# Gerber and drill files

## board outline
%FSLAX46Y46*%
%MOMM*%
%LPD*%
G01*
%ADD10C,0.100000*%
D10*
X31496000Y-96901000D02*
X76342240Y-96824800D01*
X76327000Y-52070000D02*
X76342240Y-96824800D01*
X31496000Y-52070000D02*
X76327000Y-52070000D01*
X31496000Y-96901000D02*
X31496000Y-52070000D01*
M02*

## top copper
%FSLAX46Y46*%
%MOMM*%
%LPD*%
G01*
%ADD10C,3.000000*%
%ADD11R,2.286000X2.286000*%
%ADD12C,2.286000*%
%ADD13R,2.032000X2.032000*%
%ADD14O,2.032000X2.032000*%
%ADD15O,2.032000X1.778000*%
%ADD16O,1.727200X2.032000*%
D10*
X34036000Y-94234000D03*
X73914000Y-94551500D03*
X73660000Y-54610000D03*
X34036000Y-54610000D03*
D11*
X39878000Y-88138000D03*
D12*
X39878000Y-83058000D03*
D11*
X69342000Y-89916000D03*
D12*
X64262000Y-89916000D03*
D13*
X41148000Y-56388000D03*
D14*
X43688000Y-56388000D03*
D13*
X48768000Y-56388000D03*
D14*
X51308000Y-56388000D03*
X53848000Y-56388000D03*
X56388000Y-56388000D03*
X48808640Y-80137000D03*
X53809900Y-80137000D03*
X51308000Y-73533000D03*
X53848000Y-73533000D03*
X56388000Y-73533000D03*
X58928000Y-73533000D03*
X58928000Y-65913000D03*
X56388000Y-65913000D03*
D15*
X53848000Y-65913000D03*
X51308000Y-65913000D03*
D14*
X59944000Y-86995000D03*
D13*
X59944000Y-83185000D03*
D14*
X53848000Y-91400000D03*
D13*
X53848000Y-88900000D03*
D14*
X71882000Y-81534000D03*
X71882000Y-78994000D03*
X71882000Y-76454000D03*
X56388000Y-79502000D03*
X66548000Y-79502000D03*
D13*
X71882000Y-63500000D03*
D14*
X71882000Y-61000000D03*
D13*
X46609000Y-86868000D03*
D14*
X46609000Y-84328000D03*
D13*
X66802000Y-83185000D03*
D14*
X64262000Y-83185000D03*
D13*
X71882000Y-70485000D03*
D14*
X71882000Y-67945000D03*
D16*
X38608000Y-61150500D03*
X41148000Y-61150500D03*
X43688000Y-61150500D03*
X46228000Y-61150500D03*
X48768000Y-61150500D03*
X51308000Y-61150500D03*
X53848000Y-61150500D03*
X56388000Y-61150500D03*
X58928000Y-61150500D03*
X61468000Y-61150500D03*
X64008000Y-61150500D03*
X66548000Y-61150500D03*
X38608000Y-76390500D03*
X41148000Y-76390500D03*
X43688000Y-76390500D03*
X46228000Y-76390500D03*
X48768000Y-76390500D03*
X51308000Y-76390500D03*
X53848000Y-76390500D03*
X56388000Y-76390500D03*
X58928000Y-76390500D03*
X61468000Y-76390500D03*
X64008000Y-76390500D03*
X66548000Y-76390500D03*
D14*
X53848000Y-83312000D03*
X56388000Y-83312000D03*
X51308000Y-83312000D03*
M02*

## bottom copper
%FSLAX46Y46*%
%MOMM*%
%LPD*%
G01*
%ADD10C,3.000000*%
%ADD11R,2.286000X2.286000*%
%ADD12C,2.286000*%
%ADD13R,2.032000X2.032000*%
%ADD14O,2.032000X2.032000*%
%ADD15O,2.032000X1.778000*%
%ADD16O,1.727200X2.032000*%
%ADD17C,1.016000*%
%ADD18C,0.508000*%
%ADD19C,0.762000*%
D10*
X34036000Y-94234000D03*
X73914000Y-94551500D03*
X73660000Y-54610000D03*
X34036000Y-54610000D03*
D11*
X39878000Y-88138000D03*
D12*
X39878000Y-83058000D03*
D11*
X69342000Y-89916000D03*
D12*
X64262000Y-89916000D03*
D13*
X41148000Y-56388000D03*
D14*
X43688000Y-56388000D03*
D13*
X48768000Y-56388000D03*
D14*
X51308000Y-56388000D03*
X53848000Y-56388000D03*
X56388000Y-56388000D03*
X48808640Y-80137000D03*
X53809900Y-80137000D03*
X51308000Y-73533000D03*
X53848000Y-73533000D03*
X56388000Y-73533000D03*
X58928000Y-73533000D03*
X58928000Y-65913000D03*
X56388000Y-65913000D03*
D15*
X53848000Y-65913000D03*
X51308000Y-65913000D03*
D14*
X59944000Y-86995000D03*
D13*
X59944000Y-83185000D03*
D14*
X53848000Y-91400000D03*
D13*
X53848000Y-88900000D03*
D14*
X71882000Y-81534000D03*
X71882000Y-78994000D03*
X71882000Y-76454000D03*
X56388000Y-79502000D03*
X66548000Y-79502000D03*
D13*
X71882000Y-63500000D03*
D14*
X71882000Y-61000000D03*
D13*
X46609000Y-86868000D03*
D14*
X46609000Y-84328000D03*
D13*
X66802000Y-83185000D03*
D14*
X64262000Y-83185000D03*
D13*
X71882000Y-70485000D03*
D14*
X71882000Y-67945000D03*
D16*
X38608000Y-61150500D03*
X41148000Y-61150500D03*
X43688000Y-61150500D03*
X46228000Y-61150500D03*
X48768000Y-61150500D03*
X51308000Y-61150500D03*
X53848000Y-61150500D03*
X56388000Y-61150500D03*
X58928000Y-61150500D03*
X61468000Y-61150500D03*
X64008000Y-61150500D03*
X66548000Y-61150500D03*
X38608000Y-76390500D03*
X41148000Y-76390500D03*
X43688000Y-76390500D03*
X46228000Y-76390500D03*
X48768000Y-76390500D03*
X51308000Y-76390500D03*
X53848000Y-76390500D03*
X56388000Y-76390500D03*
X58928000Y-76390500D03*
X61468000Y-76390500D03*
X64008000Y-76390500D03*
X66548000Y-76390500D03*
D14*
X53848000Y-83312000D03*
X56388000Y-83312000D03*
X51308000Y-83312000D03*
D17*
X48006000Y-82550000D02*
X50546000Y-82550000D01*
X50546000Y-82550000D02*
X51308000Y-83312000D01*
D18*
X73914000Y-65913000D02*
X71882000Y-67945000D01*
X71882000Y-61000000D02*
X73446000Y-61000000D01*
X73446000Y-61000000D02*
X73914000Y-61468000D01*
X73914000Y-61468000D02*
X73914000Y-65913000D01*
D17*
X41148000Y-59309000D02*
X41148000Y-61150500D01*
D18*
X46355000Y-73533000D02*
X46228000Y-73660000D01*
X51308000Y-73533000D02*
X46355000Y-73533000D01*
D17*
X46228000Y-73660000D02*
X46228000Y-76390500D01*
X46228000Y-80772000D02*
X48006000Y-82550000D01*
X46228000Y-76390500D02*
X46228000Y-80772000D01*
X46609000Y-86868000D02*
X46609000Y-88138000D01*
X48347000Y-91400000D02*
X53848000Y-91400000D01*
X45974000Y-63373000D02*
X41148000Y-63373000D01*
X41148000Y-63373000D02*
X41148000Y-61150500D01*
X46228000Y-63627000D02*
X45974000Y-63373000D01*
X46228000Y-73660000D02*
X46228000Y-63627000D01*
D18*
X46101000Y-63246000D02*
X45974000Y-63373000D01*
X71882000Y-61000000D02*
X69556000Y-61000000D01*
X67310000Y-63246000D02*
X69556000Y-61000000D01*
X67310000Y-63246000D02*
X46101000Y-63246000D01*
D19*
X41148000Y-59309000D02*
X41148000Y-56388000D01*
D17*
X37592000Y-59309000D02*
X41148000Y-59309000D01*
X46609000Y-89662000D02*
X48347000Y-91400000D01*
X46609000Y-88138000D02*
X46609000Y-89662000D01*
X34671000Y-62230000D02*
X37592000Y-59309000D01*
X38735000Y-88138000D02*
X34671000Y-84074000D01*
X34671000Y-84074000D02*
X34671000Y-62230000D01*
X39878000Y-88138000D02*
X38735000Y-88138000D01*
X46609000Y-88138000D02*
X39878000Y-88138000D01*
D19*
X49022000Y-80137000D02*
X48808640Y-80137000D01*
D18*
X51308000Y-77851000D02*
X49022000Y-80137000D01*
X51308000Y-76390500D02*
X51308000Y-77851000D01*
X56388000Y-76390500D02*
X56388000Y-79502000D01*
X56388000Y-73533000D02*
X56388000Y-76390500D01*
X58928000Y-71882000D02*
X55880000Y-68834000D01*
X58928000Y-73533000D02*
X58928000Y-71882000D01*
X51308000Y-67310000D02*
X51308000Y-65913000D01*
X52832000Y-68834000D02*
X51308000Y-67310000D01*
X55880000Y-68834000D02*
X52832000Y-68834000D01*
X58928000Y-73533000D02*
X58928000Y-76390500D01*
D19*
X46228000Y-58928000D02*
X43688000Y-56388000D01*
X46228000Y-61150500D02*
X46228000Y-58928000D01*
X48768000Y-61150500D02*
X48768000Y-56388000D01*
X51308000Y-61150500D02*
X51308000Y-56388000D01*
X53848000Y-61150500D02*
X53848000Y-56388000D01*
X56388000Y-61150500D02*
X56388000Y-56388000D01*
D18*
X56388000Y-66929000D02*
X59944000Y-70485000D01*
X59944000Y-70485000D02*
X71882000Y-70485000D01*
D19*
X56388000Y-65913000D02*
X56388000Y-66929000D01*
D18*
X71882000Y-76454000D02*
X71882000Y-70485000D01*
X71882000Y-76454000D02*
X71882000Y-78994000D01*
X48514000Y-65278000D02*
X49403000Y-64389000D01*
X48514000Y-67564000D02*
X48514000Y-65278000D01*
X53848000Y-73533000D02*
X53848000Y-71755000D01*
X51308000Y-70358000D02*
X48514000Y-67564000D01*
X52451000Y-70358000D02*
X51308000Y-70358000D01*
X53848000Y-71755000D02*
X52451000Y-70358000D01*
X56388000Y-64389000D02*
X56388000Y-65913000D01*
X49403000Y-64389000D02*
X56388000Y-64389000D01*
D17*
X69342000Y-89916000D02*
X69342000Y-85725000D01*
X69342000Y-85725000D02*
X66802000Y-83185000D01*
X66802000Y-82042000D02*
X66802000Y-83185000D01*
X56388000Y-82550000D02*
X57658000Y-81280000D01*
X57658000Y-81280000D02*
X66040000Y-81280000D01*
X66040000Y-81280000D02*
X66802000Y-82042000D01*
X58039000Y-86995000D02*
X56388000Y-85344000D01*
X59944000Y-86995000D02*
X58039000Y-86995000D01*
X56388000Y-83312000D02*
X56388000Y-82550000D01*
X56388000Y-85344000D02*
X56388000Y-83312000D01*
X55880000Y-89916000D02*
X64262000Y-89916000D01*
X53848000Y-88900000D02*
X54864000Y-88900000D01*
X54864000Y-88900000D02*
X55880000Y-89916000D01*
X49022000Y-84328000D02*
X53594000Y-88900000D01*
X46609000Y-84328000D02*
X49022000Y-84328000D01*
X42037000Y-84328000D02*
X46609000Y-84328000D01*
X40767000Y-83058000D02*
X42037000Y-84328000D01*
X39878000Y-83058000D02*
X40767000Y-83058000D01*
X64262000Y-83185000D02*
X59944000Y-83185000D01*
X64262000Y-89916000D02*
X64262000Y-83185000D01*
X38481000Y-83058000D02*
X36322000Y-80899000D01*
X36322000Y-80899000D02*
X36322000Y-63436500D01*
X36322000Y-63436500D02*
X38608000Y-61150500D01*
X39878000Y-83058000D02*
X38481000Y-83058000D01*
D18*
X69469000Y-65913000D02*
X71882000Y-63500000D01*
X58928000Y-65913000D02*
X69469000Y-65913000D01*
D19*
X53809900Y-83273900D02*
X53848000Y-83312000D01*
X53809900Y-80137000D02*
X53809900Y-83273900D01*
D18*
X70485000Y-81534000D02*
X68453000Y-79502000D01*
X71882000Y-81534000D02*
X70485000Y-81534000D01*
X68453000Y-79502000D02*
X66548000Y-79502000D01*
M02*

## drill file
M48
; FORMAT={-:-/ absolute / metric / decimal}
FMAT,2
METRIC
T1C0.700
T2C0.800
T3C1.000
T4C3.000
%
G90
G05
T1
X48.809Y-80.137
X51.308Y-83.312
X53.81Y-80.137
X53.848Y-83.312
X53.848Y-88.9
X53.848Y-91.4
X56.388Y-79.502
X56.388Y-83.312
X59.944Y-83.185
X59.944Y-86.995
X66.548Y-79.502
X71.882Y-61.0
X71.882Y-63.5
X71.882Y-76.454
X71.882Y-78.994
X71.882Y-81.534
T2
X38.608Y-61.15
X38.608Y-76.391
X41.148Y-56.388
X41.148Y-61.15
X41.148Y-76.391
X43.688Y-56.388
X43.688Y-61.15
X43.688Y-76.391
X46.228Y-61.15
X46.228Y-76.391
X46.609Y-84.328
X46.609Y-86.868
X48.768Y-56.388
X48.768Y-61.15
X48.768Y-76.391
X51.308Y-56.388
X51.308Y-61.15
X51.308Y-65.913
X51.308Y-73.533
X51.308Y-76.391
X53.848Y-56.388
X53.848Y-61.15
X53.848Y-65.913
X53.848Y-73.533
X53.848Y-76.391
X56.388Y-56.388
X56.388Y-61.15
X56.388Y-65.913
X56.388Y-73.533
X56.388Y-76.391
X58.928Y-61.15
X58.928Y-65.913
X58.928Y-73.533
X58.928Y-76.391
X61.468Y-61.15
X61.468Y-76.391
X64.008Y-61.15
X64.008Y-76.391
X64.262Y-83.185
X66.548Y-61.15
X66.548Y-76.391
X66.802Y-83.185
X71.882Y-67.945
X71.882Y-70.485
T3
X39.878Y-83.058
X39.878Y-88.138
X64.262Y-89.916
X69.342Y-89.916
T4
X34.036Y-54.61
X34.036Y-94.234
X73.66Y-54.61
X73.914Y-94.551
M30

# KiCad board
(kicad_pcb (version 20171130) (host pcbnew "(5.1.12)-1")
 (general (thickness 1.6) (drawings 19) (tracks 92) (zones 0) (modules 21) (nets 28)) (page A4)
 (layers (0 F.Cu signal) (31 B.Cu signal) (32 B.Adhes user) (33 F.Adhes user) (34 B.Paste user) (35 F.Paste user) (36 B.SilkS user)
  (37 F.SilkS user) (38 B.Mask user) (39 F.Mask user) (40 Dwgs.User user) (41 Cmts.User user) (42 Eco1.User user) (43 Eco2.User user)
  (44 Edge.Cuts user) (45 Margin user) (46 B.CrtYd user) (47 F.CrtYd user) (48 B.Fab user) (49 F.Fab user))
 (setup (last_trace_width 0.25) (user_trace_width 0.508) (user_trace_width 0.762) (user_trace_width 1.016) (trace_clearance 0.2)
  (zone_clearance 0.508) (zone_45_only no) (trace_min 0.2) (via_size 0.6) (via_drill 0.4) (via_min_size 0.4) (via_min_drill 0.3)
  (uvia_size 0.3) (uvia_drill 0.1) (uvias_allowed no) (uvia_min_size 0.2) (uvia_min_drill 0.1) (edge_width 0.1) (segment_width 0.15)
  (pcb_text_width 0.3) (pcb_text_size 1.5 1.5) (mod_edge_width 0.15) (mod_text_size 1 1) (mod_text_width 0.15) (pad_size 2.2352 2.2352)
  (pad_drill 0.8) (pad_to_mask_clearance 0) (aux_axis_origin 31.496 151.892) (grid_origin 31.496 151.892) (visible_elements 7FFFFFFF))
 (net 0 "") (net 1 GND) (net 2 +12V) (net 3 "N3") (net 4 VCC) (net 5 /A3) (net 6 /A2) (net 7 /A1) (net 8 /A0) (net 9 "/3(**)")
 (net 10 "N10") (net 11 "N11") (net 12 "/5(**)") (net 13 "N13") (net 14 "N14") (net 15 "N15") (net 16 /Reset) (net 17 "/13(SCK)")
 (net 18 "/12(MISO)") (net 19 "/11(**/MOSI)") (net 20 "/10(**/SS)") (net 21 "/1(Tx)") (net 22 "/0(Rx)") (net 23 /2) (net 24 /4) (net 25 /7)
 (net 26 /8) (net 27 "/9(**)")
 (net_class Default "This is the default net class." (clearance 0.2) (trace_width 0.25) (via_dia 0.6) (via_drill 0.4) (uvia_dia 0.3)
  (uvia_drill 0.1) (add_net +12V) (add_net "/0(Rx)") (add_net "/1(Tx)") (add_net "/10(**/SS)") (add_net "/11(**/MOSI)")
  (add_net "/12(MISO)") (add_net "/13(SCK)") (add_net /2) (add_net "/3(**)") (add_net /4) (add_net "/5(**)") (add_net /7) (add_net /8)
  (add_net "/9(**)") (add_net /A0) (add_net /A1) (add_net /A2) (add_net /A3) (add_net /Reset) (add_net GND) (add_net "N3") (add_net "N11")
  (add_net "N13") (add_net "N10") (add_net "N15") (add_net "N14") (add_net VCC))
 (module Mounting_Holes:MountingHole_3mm (layer F.Cu) (at 34.036 94.234)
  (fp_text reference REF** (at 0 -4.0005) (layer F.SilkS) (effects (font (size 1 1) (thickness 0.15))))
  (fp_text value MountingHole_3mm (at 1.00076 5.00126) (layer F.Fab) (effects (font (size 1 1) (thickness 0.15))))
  (pad 1 thru_hole circle (at 0 0) (size 3 3) (drill 3) (layers)))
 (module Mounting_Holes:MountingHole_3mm (layer F.Cu) (at 73.914 94.5515)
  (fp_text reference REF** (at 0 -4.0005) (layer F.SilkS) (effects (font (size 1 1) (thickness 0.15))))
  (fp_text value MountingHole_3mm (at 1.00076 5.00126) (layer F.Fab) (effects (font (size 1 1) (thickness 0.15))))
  (pad 1 thru_hole circle (at 0 0) (size 3 3) (drill 3) (layers)))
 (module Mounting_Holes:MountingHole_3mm (layer F.Cu) (at 73.66 54.61)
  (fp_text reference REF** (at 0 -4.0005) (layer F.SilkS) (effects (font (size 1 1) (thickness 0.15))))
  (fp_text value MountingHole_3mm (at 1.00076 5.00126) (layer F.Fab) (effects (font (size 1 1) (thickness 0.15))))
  (pad 1 thru_hole circle (at 0 0) (size 3 3) (drill 3) (layers)))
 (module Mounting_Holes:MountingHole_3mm (layer F.Cu) (at 34.036 54.61)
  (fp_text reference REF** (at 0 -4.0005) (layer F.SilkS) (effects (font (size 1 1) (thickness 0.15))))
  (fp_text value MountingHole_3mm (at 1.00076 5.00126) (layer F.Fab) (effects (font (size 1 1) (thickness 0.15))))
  (pad 1 thru_hole circle (at 0 0) (size 3 3) (drill 3) (layers)))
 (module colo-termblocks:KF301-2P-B (layer F.Cu) (at 39.878 85.598 90)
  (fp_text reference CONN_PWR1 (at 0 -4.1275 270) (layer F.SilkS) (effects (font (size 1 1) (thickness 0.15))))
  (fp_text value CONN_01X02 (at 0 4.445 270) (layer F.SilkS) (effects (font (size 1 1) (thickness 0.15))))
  (pad 1 thru_hole rect (at -2.54 0 90) (size 2.286 2.286) (drill 1) (layers B.Cu B.Mask) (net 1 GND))
  (pad 2 thru_hole circle (at 2.54 0 90) (size 2.286 2.286) (drill 1) (layers B.Cu B.Mask) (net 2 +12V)))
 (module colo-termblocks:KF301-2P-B (layer F.Cu) (at 66.802 89.916 180)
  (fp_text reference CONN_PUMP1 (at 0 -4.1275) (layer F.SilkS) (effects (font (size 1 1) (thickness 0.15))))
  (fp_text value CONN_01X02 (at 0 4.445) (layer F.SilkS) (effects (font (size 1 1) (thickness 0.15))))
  (pad 1 thru_hole rect (at -2.54 0 180) (size 2.286 2.286) (drill 1) (layers B.Cu B.Mask) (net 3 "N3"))
  (pad 2 thru_hole circle (at 2.54 0 180) (size 2.286 2.286) (drill 1) (layers B.Cu B.Mask) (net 2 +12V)))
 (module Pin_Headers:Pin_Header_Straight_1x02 (layer F.Cu) (at 41.148 56.388 90)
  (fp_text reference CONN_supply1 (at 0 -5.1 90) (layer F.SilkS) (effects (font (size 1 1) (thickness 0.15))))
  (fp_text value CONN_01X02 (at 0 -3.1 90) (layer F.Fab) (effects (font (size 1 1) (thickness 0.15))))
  (pad 1 thru_hole rect (at 0 0 90) (size 2.032 2.032) (drill 0.8) (layers B.Cu B.Mask) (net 1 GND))
  (pad 2 thru_hole oval (at 0 2.54 90) (size 2.032 2.032) (drill 0.8) (layers B.Cu B.Mask) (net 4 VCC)))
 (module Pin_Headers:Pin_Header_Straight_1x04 (layer F.Cu) (at 48.768 56.388 90)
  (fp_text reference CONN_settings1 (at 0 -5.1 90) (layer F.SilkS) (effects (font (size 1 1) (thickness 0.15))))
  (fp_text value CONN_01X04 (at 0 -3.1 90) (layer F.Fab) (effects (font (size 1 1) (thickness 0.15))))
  (pad 1 thru_hole rect (at 0 0 90) (size 2.032 2.032) (drill 0.8) (layers B.Cu B.Mask) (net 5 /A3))
  (pad 2 thru_hole oval (at 0 2.54 90) (size 2.032 2.032) (drill 0.8) (layers B.Cu B.Mask) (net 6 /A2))
  (pad 3 thru_hole oval (at 0 5.08 90) (size 2.032 2.032) (drill 0.8) (layers B.Cu B.Mask) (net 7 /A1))
  (pad 4 thru_hole oval (at 0 7.62 90) (size 2.032 2.032) (drill 0.8) (layers B.Cu B.Mask) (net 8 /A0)))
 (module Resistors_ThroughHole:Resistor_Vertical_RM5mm (layer F.Cu) (at 51.308 80.137)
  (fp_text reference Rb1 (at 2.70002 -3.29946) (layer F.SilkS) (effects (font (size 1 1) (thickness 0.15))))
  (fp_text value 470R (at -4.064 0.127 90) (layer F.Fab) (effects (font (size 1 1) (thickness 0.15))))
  (pad 1 thru_hole oval (at -2.49936 0) (size 2.032 2.032) (drill 0.7) (layers B.Cu B.Mask) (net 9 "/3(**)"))
  (pad 2 thru_hole oval (at 2.5019 0) (size 2.032 2.032) (drill 0.7) (layers B.Cu B.Mask) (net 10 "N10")))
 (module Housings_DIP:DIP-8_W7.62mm (layer F.Cu) (at 51.308 73.533 90)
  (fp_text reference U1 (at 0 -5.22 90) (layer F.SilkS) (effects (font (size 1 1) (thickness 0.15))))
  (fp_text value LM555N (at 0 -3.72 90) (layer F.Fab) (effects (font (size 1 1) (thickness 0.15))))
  (pad 1 thru_hole oval (at 0 0 90) (size 2.032 2.032) (drill 0.8) (layers B.Cu B.Mask) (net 1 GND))
  (pad 2 thru_hole oval (at 0 2.54 90) (size 2.032 2.032) (drill 0.8) (layers B.Cu B.Mask) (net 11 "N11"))
  (pad 3 thru_hole oval (at 0 5.08 90) (size 2.032 2.032) (drill 0.8) (layers B.Cu B.Mask) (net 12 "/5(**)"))
  (pad 4 thru_hole oval (at 0 7.62 90) (size 2.032 2.032) (drill 0.8) (layers B.Cu B.Mask) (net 4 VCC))
  (pad 5 thru_hole oval (at 7.62 7.62 90) (size 2.032 2.032) (drill 0.8) (layers B.Cu B.Mask) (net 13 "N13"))
  (pad 6 thru_hole oval (at 7.62 5.08 90) (size 2.032 2.032) (drill 0.8) (layers B.Cu B.Mask) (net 11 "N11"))
  (pad 7 thru_hole oval (at 7.62 2.54 90) (size 1.778 2.032) (drill 0.8) (layers B.Cu B.Mask) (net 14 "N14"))
  (pad 8 thru_hole oval (at 7.62 0 90) (size 1.778 2.032) (drill 0.8) (layers B.Cu B.Mask) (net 4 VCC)))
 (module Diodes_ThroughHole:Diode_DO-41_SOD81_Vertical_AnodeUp (layer F.Cu) (at 59.944 83.185 270)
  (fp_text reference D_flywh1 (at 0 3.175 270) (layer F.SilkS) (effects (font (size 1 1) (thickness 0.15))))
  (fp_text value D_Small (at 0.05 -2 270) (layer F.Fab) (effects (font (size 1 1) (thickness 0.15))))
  (pad 2 thru_hole oval (at 3.81 0 270) (size 2.032 2.032) (drill 0.7) (layers B.Cu B.Mask) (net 3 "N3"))
  (pad 1 thru_hole rect (at 0 0 270) (size 2.032 2.032) (drill 0.7) (layers B.Cu B.Mask) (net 2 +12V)))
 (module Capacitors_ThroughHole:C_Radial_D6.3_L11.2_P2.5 (layer F.Cu) (at 53.848 88.9 270)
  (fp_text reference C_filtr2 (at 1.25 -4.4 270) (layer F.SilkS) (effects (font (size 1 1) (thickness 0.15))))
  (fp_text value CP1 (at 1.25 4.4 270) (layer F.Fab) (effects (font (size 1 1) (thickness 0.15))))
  (pad 2 thru_hole oval (at 2.5 0 270) (size 2.032 2.032) (drill 0.7) (layers B.Cu B.Mask) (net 1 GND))
  (pad 1 thru_hole rect (at 0 0 270) (size 2.032 2.032) (drill 0.7) (layers B.Cu B.Mask) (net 2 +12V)))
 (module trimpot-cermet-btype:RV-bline (layer F.Cu) (at 71.882 78.994 90)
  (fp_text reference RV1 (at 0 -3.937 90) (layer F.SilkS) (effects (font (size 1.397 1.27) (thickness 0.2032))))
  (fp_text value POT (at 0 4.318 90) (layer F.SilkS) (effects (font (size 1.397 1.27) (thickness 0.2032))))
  (pad 1 thru_hole oval (at -2.54 0 90) (size 2.032 2.032) (drill 0.7) (layers B.Cu B.Mask) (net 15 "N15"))
  (pad 2 thru_hole oval (at 0 0 90) (size 2.032 2.032) (drill 0.7) (layers B.Cu B.Mask) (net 11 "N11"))
  (pad 3 thru_hole oval (at 2.54 0 90) (size 2.032 2.032) (drill 0.7) (layers B.Cu B.Mask) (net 11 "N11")))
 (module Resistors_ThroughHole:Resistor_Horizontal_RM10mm (layer F.Cu) (at 61.468 79.502)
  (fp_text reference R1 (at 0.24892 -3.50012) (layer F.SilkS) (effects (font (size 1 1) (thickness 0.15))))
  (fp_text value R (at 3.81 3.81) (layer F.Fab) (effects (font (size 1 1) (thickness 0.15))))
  (pad 1 thru_hole oval (at -5.08 0) (size 2.032 2.032) (drill 0.7) (layers B.Cu B.Mask) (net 12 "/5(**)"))
  (pad 2 thru_hole oval (at 5.08 0) (size 2.032 2.032) (drill 0.7) (layers B.Cu B.Mask) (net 15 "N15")))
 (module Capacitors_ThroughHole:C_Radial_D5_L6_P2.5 (layer F.Cu) (at 71.882 63.5 90)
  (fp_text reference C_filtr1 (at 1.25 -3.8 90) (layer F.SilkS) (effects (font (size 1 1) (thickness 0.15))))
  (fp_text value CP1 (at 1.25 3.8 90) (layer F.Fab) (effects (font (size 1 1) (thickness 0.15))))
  (pad 1 thru_hole rect (at 0 0 90) (size 2.032 2.032) (drill 0.7) (layers B.Cu B.Mask) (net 13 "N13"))
  (pad 2 thru_hole oval (at 2.5 0 90) (size 2.032 2.032) (drill 0.7) (layers B.Cu B.Mask) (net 1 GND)))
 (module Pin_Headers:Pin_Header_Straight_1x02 (layer F.Cu) (at 46.609 86.868 180)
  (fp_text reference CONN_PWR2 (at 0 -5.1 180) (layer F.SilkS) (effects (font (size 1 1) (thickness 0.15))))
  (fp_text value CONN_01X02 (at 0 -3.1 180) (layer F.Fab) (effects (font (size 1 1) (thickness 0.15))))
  (pad 1 thru_hole rect (at 0 0 180) (size 2.032 2.032) (drill 0.8) (layers B.Cu B.Mask) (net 1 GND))
  (pad 2 thru_hole oval (at 0 2.54 180) (size 2.032 2.032) (drill 0.8) (layers B.Cu B.Mask) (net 2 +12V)))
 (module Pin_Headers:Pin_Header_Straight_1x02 (layer F.Cu) (at 66.802 83.185 270)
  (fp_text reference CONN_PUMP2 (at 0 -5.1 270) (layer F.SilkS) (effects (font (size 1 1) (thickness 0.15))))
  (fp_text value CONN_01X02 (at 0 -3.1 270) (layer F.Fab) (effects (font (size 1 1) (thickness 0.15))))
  (pad 1 thru_hole rect (at 0 0 270) (size 2.032 2.032) (drill 0.8) (layers B.Cu B.Mask) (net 3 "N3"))
  (pad 2 thru_hole oval (at 0 2.54 270) (size 2.032 2.032) (drill 0.8) (layers B.Cu B.Mask) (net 2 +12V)))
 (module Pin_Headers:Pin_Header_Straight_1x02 (layer F.Cu) (at 71.882 70.485 180)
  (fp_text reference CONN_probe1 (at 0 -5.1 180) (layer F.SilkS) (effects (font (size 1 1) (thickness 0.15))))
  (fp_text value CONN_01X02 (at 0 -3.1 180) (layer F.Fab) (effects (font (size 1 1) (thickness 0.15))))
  (pad 1 thru_hole rect (at 0 0 180) (size 2.032 2.032) (drill 0.8) (layers B.Cu B.Mask) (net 11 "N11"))
  (pad 2 thru_hole oval (at 0 2.54 180) (size 2.032 2.032) (drill 0.8) (layers B.Cu B.Mask) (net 1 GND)))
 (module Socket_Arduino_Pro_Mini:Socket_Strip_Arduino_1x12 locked (layer F.Cu) (at 38.608 61.1505)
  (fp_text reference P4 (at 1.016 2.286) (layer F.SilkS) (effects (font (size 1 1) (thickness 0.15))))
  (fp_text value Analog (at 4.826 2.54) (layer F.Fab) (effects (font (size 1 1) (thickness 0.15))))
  (pad 1 thru_hole oval (at 0 0) (size 1.7272 2.032) (drill 0.8) (layers B.Cu B.Mask) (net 2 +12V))
  (pad 2 thru_hole oval (at 2.54 0) (size 1.7272 2.032) (drill 0.8) (layers B.Cu B.Mask) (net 1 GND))
  (pad 3 thru_hole oval (at 5.08 0) (size 1.7272 2.032) (drill 0.8) (layers B.Cu B.Mask) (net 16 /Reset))
  (pad 4 thru_hole oval (at 7.62 0) (size 1.7272 2.032) (drill 0.8) (layers B.Cu B.Mask) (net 4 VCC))
  (pad 5 thru_hole oval (at 10.16 0) (size 1.7272 2.032) (drill 0.8) (layers B.Cu B.Mask) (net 5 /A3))
  (pad 6 thru_hole oval (at 12.7 0) (size 1.7272 2.032) (drill 0.8) (layers B.Cu B.Mask) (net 6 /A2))
  (pad 7 thru_hole oval (at 15.24 0) (size 1.7272 2.032) (drill 0.8) (layers B.Cu B.Mask) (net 7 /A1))
  (pad 8 thru_hole oval (at 17.78 0) (size 1.7272 2.032) (drill 0.8) (layers B.Cu B.Mask) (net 8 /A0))
  (pad 9 thru_hole oval (at 20.32 0) (size 1.7272 2.032) (drill 0.8) (layers B.Cu B.Mask) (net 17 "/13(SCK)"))
  (pad 10 thru_hole oval (at 22.86 0) (size 1.7272 2.032) (drill 0.8) (layers B.Cu B.Mask) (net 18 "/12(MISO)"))
  (pad 11 thru_hole oval (at 25.4 0) (size 1.7272 2.032) (drill 0.8) (layers B.Cu B.Mask) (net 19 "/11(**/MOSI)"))
  (pad 12 thru_hole oval (at 27.94 0) (size 1.7272 2.032) (drill 0.8) (layers B.Cu B.Mask) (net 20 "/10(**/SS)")))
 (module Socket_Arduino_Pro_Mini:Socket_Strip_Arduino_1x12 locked (layer F.Cu) (at 38.608 76.3905)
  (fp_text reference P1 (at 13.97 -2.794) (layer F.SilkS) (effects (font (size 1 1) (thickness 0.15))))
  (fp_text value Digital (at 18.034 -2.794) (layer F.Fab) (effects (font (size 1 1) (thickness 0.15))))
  (pad 1 thru_hole oval (at 0 0) (size 1.7272 2.032) (drill 0.8) (layers B.Cu B.Mask) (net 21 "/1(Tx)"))
  (pad 2 thru_hole oval (at 2.54 0) (size 1.7272 2.032) (drill 0.8) (layers B.Cu B.Mask) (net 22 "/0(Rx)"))
  (pad 3 thru_hole oval (at 5.08 0) (size 1.7272 2.032) (drill 0.8) (layers B.Cu B.Mask) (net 16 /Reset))
  (pad 4 thru_hole oval (at 7.62 0) (size 1.7272 2.032) (drill 0.8) (layers B.Cu B.Mask) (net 1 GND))
  (pad 5 thru_hole oval (at 10.16 0) (size 1.7272 2.032) (drill 0.8) (layers B.Cu B.Mask) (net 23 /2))
  (pad 6 thru_hole oval (at 12.7 0) (size 1.7272 2.032) (drill 0.8) (layers B.Cu B.Mask) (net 9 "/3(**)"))
  (pad 7 thru_hole oval (at 15.24 0) (size 1.7272 2.032) (drill 0.8) (layers B.Cu B.Mask) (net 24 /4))
  (pad 8 thru_hole oval (at 17.78 0) (size 1.7272 2.032) (drill 0.8) (layers B.Cu B.Mask) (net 12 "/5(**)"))
  (pad 9 thru_hole oval (at 20.32 0) (size 1.7272 2.032) (drill 0.8) (layers B.Cu B.Mask) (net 4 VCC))
  (pad 10 thru_hole oval (at 22.86 0) (size 1.7272 2.032) (drill 0.8) (layers B.Cu B.Mask) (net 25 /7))
  (pad 11 thru_hole oval (at 25.4 0) (size 1.7272 2.032) (drill 0.8) (layers B.Cu B.Mask) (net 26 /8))
  (pad 12 thru_hole oval (at 27.94 0) (size 1.7272 2.032) (drill 0.8) (layers B.Cu B.Mask) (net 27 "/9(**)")))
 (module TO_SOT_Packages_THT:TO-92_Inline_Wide (layer F.Cu) (at 51.308 83.312)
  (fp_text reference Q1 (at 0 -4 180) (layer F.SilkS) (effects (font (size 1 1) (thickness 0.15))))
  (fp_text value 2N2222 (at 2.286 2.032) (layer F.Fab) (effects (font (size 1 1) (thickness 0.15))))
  (pad 2 thru_hole oval (at 2.54 0) (size 2.032 2.032) (drill 0.7) (layers B.Cu B.Mask) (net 10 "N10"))
  (pad 3 thru_hole oval (at 5.08 0) (size 2.032 2.032) (drill 0.7) (layers B.Cu B.Mask) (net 3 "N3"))
  (pad 1 thru_hole oval (at 0 0) (size 2.032 2.032) (drill 0.7) (layers B.Cu B.Mask) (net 1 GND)))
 (gr_line (start 31.496 96.901) (end 76.34224 96.8248) (angle 90) (layer Edge.Cuts) (width 0.1))
 (gr_line (start 76.327 52.07) (end 76.34224 96.8248) (angle 90) (layer Edge.Cuts) (width 0.1))
 (gr_line (start 31.496 52.07) (end 76.327 52.07) (angle 90) (layer Edge.Cuts) (width 0.1))
 (gr_line (start 31.496 96.901) (end 31.496 52.07) (angle 90) (layer Edge.Cuts) (width 0.1))
 (segment (start 48.006 82.55) (end 50.546 82.55) (width 1.016) (layer B.Cu) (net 1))
 (segment (start 50.546 82.55) (end 51.308 83.312) (width 1.016) (layer B.Cu) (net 1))
 (segment (start 73.914 65.913) (end 71.882 67.945) (width 0.508) (layer B.Cu) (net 1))
 (segment (start 71.882 61) (end 73.446 61) (width 0.508) (layer B.Cu) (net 1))
 (segment (start 73.446 61) (end 73.914 61.468) (width 0.508) (layer B.Cu) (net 1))
 (segment (start 73.914 61.468) (end 73.914 65.913) (width 0.508) (layer B.Cu) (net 1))
 (segment (start 41.148 59.309) (end 41.148 61.1505) (width 1.016) (layer B.Cu) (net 1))
 (segment (start 46.355 73.533) (end 46.228 73.66) (width 0.508) (layer B.Cu) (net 1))
 (segment (start 51.308 73.533) (end 46.355 73.533) (width 0.508) (layer B.Cu) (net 1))
 (segment (start 46.228 73.66) (end 46.228 76.3905) (width 1.016) (layer B.Cu) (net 1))
 (segment (start 46.228 80.772) (end 48.006 82.55) (width 1.016) (layer B.Cu) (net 1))
 (segment (start 46.228 76.3905) (end 46.228 80.772) (width 1.016) (layer B.Cu) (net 1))
 (segment (start 46.609 86.868) (end 46.609 88.138) (width 1.016) (layer B.Cu) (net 1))
 (segment (start 48.347 91.4) (end 53.848 91.4) (width 1.016) (layer B.Cu) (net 1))
 (segment (start 45.974 63.373) (end 41.148 63.373) (width 1.016) (layer B.Cu) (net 1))
 (segment (start 41.148 63.373) (end 41.148 61.1505) (width 1.016) (layer B.Cu) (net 1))
 (segment (start 46.228 63.627) (end 45.974 63.373) (width 1.016) (layer B.Cu) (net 1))
 (segment (start 46.228 73.66) (end 46.228 63.627) (width 1.016) (layer B.Cu) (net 1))
 (segment (start 46.101 63.246) (end 45.974 63.373) (width 0.508) (layer B.Cu) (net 1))
 (segment (start 71.882 61) (end 69.556 61) (width 0.508) (layer B.Cu) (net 1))
 (segment (start 67.31 63.246) (end 69.556 61) (width 0.508) (layer B.Cu) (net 1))
 (segment (start 67.31 63.246) (end 46.101 63.246) (width 0.508) (layer B.Cu) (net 1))
 (segment (start 41.148 59.309) (end 41.148 56.388) (width 0.762) (layer B.Cu) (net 1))
 (segment (start 37.592 59.309) (end 41.148 59.309) (width 1.016) (layer B.Cu) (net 1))
 (segment (start 46.609 89.662) (end 48.347 91.4) (width 1.016) (layer B.Cu) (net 1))
 (segment (start 46.609 88.138) (end 46.609 89.662) (width 1.016) (layer B.Cu) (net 1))
 (segment (start 34.671 62.23) (end 37.592 59.309) (width 1.016) (layer B.Cu) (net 1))
 (segment (start 38.735 88.138) (end 34.671 84.074) (width 1.016) (layer B.Cu) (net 1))
 (segment (start 34.671 84.074) (end 34.671 62.23) (width 1.016) (layer B.Cu) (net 1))
 (segment (start 39.878 88.138) (end 38.735 88.138) (width 1.016) (layer B.Cu) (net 1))
 (segment (start 46.609 88.138) (end 39.878 88.138) (width 1.016) (layer B.Cu) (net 1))
 (segment (start 49.022 80.137) (end 48.80864 80.137) (width 0.762) (layer B.Cu) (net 9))
 (segment (start 51.308 77.851) (end 49.022 80.137) (width 0.508) (layer B.Cu) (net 9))
 (segment (start 51.308 76.3905) (end 51.308 77.851) (width 0.508) (layer B.Cu) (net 9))
 (segment (start 56.388 76.3905) (end 56.388 79.502) (width 0.508) (layer B.Cu) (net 12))
 (segment (start 56.388 73.533) (end 56.388 76.3905) (width 0.508) (layer B.Cu) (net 12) (status 10))
 (segment (start 58.928 71.882) (end 55.88 68.834) (width 0.508) (layer B.Cu) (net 4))
 (segment (start 58.928 73.533) (end 58.928 71.882) (width 0.508) (layer B.Cu) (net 4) (status 10))
 (segment (start 51.308 67.31) (end 51.308 65.913) (width 0.508) (layer B.Cu) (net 4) (status 20))
 (segment (start 52.832 68.834) (end 51.308 67.31) (width 0.508) (layer B.Cu) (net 4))
 (segment (start 55.88 68.834) (end 52.832 68.834) (width 0.508) (layer B.Cu) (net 4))
 (segment (start 58.928 73.533) (end 58.928 76.3905) (width 0.508) (layer B.Cu) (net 4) (status 10))
 (segment (start 46.228 58.928) (end 43.688 56.388) (width 0.762) (layer B.Cu) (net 4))
 (segment (start 46.228 61.1505) (end 46.228 58.928) (width 0.762) (layer B.Cu) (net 4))
 (segment (start 48.768 61.1505) (end 48.768 56.388) (width 0.762) (layer B.Cu) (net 5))
 (segment (start 51.308 61.1505) (end 51.308 56.388) (width 0.762) (layer B.Cu) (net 6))
 (segment (start 53.848 61.1505) (end 53.848 56.388) (width 0.762) (layer B.Cu) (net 7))
 (segment (start 56.388 61.1505) (end 56.388 56.388) (width 0.762) (layer B.Cu) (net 8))
 (segment (start 56.388 66.929) (end 59.944 70.485) (width 0.508) (layer B.Cu) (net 11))
 (segment (start 59.944 70.485) (end 71.882 70.485) (width 0.508) (layer B.Cu) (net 11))
 (segment (start 56.388 65.913) (end 56.388 66.929) (width 0.762) (layer B.Cu) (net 11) (status 10))
 (segment (start 71.882 76.454) (end 71.882 70.485) (width 0.508) (layer B.Cu) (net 11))
 (segment (start 71.882 76.454) (end 71.882 78.994) (width 0.508) (layer B.Cu) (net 11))
 (segment (start 48.514 65.278) (end 49.403 64.389) (width 0.508) (layer B.Cu) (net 11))
 (segment (start 48.514 67.564) (end 48.514 65.278) (width 0.508) (layer B.Cu) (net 11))
 (segment (start 53.848 73.533) (end 53.848 71.755) (width 0.508) (layer B.Cu) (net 11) (status 10))
 (segment (start 51.308 70.358) (end 48.514 67.564) (width 0.508) (layer B.Cu) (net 11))
 (segment (start 52.451 70.358) (end 51.308 70.358) (width 0.508) (layer B.Cu) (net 11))
 (segment (start 53.848 71.755) (end 52.451 70.358) (width 0.508) (layer B.Cu) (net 11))
 (segment (start 56.388 64.389) (end 56.388 65.913) (width 0.508) (layer B.Cu) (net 11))
 (segment (start 49.403 64.389) (end 56.388 64.389) (width 0.508) (layer B.Cu) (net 11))
 (segment (start 69.342 89.916) (end 69.342 85.725) (width 1.016) (layer B.Cu) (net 3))
 (segment (start 69.342 85.725) (end 66.802 83.185) (width 1.016) (layer B.Cu) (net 3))
 (segment (start 66.802 82.042) (end 66.802 83.185) (width 1.016) (layer B.Cu) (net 3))
 (segment (start 56.388 82.55) (end 57.658 81.28) (width 1.016) (layer B.Cu) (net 3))
 (segment (start 57.658 81.28) (end 66.04 81.28) (width 1.016) (layer B.Cu) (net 3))
 (segment (start 66.04 81.28) (end 66.802 82.042) (width 1.016) (layer B.Cu) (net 3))
 (segment (start 58.039 86.995) (end 56.388 85.344) (width 1.016) (layer B.Cu) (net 3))
 (segment (start 59.944 86.995) (end 58.039 86.995) (width 1.016) (layer B.Cu) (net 3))
 (segment (start 56.388 83.312) (end 56.388 82.55) (width 1.016) (layer B.Cu) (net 3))
 (segment (start 56.388 85.344) (end 56.388 83.312) (width 1.016) (layer B.Cu) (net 3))
 (segment (start 55.88 89.916) (end 64.262 89.916) (width 1.016) (layer B.Cu) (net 2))
 (segment (start 53.848 88.9) (end 54.864 88.9) (width 1.016) (layer B.Cu) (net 2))
 (segment (start 54.864 88.9) (end 55.88 89.916) (width 1.016) (layer B.Cu) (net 2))
 (segment (start 49.022 84.328) (end 53.594 88.9) (width 1.016) (layer B.Cu) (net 2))
 (segment (start 46.609 84.328) (end 49.022 84.328) (width 1.016) (layer B.Cu) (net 2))
 (segment (start 42.037 84.328) (end 46.609 84.328) (width 1.016) (layer B.Cu) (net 2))
 (segment (start 40.767 83.058) (end 42.037 84.328) (width 1.016) (layer B.Cu) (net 2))
 (segment (start 39.878 83.058) (end 40.767 83.058) (width 1.016) (layer B.Cu) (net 2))
 (segment (start 64.262 83.185) (end 59.944 83.185) (width 1.016) (layer B.Cu) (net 2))
 (segment (start 64.262 89.916) (end 64.262 83.185) (width 1.016) (layer B.Cu) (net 2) (status 10))
 (segment (start 38.481 83.058) (end 36.322 80.899) (width 1.016) (layer B.Cu) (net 2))
 (segment (start 36.322 80.899) (end 36.322 63.4365) (width 1.016) (layer B.Cu) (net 2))
 (segment (start 36.322 63.4365) (end 38.608 61.1505) (width 1.016) (layer B.Cu) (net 2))
 (segment (start 39.878 83.058) (end 38.481 83.058) (width 1.016) (layer B.Cu) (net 2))
 (segment (start 69.469 65.913) (end 71.882 63.5) (width 0.508) (layer B.Cu) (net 13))
 (segment (start 58.928 65.913) (end 69.469 65.913) (width 0.508) (layer B.Cu) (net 13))
 (segment (start 53.8099 83.2739) (end 53.848 83.312) (width 0.762) (layer B.Cu) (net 10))
 (segment (start 53.8099 80.137) (end 53.8099 83.2739) (width 0.762) (layer B.Cu) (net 10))
 (segment (start 70.485 81.534) (end 68.453 79.502) (width 0.508) (layer B.Cu) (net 15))
 (segment (start 71.882 81.534) (end 70.485 81.534) (width 0.508) (layer B.Cu) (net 15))
 (segment (start 68.453 79.502) (end 66.548 79.502) (width 0.508) (layer B.Cu) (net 15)))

